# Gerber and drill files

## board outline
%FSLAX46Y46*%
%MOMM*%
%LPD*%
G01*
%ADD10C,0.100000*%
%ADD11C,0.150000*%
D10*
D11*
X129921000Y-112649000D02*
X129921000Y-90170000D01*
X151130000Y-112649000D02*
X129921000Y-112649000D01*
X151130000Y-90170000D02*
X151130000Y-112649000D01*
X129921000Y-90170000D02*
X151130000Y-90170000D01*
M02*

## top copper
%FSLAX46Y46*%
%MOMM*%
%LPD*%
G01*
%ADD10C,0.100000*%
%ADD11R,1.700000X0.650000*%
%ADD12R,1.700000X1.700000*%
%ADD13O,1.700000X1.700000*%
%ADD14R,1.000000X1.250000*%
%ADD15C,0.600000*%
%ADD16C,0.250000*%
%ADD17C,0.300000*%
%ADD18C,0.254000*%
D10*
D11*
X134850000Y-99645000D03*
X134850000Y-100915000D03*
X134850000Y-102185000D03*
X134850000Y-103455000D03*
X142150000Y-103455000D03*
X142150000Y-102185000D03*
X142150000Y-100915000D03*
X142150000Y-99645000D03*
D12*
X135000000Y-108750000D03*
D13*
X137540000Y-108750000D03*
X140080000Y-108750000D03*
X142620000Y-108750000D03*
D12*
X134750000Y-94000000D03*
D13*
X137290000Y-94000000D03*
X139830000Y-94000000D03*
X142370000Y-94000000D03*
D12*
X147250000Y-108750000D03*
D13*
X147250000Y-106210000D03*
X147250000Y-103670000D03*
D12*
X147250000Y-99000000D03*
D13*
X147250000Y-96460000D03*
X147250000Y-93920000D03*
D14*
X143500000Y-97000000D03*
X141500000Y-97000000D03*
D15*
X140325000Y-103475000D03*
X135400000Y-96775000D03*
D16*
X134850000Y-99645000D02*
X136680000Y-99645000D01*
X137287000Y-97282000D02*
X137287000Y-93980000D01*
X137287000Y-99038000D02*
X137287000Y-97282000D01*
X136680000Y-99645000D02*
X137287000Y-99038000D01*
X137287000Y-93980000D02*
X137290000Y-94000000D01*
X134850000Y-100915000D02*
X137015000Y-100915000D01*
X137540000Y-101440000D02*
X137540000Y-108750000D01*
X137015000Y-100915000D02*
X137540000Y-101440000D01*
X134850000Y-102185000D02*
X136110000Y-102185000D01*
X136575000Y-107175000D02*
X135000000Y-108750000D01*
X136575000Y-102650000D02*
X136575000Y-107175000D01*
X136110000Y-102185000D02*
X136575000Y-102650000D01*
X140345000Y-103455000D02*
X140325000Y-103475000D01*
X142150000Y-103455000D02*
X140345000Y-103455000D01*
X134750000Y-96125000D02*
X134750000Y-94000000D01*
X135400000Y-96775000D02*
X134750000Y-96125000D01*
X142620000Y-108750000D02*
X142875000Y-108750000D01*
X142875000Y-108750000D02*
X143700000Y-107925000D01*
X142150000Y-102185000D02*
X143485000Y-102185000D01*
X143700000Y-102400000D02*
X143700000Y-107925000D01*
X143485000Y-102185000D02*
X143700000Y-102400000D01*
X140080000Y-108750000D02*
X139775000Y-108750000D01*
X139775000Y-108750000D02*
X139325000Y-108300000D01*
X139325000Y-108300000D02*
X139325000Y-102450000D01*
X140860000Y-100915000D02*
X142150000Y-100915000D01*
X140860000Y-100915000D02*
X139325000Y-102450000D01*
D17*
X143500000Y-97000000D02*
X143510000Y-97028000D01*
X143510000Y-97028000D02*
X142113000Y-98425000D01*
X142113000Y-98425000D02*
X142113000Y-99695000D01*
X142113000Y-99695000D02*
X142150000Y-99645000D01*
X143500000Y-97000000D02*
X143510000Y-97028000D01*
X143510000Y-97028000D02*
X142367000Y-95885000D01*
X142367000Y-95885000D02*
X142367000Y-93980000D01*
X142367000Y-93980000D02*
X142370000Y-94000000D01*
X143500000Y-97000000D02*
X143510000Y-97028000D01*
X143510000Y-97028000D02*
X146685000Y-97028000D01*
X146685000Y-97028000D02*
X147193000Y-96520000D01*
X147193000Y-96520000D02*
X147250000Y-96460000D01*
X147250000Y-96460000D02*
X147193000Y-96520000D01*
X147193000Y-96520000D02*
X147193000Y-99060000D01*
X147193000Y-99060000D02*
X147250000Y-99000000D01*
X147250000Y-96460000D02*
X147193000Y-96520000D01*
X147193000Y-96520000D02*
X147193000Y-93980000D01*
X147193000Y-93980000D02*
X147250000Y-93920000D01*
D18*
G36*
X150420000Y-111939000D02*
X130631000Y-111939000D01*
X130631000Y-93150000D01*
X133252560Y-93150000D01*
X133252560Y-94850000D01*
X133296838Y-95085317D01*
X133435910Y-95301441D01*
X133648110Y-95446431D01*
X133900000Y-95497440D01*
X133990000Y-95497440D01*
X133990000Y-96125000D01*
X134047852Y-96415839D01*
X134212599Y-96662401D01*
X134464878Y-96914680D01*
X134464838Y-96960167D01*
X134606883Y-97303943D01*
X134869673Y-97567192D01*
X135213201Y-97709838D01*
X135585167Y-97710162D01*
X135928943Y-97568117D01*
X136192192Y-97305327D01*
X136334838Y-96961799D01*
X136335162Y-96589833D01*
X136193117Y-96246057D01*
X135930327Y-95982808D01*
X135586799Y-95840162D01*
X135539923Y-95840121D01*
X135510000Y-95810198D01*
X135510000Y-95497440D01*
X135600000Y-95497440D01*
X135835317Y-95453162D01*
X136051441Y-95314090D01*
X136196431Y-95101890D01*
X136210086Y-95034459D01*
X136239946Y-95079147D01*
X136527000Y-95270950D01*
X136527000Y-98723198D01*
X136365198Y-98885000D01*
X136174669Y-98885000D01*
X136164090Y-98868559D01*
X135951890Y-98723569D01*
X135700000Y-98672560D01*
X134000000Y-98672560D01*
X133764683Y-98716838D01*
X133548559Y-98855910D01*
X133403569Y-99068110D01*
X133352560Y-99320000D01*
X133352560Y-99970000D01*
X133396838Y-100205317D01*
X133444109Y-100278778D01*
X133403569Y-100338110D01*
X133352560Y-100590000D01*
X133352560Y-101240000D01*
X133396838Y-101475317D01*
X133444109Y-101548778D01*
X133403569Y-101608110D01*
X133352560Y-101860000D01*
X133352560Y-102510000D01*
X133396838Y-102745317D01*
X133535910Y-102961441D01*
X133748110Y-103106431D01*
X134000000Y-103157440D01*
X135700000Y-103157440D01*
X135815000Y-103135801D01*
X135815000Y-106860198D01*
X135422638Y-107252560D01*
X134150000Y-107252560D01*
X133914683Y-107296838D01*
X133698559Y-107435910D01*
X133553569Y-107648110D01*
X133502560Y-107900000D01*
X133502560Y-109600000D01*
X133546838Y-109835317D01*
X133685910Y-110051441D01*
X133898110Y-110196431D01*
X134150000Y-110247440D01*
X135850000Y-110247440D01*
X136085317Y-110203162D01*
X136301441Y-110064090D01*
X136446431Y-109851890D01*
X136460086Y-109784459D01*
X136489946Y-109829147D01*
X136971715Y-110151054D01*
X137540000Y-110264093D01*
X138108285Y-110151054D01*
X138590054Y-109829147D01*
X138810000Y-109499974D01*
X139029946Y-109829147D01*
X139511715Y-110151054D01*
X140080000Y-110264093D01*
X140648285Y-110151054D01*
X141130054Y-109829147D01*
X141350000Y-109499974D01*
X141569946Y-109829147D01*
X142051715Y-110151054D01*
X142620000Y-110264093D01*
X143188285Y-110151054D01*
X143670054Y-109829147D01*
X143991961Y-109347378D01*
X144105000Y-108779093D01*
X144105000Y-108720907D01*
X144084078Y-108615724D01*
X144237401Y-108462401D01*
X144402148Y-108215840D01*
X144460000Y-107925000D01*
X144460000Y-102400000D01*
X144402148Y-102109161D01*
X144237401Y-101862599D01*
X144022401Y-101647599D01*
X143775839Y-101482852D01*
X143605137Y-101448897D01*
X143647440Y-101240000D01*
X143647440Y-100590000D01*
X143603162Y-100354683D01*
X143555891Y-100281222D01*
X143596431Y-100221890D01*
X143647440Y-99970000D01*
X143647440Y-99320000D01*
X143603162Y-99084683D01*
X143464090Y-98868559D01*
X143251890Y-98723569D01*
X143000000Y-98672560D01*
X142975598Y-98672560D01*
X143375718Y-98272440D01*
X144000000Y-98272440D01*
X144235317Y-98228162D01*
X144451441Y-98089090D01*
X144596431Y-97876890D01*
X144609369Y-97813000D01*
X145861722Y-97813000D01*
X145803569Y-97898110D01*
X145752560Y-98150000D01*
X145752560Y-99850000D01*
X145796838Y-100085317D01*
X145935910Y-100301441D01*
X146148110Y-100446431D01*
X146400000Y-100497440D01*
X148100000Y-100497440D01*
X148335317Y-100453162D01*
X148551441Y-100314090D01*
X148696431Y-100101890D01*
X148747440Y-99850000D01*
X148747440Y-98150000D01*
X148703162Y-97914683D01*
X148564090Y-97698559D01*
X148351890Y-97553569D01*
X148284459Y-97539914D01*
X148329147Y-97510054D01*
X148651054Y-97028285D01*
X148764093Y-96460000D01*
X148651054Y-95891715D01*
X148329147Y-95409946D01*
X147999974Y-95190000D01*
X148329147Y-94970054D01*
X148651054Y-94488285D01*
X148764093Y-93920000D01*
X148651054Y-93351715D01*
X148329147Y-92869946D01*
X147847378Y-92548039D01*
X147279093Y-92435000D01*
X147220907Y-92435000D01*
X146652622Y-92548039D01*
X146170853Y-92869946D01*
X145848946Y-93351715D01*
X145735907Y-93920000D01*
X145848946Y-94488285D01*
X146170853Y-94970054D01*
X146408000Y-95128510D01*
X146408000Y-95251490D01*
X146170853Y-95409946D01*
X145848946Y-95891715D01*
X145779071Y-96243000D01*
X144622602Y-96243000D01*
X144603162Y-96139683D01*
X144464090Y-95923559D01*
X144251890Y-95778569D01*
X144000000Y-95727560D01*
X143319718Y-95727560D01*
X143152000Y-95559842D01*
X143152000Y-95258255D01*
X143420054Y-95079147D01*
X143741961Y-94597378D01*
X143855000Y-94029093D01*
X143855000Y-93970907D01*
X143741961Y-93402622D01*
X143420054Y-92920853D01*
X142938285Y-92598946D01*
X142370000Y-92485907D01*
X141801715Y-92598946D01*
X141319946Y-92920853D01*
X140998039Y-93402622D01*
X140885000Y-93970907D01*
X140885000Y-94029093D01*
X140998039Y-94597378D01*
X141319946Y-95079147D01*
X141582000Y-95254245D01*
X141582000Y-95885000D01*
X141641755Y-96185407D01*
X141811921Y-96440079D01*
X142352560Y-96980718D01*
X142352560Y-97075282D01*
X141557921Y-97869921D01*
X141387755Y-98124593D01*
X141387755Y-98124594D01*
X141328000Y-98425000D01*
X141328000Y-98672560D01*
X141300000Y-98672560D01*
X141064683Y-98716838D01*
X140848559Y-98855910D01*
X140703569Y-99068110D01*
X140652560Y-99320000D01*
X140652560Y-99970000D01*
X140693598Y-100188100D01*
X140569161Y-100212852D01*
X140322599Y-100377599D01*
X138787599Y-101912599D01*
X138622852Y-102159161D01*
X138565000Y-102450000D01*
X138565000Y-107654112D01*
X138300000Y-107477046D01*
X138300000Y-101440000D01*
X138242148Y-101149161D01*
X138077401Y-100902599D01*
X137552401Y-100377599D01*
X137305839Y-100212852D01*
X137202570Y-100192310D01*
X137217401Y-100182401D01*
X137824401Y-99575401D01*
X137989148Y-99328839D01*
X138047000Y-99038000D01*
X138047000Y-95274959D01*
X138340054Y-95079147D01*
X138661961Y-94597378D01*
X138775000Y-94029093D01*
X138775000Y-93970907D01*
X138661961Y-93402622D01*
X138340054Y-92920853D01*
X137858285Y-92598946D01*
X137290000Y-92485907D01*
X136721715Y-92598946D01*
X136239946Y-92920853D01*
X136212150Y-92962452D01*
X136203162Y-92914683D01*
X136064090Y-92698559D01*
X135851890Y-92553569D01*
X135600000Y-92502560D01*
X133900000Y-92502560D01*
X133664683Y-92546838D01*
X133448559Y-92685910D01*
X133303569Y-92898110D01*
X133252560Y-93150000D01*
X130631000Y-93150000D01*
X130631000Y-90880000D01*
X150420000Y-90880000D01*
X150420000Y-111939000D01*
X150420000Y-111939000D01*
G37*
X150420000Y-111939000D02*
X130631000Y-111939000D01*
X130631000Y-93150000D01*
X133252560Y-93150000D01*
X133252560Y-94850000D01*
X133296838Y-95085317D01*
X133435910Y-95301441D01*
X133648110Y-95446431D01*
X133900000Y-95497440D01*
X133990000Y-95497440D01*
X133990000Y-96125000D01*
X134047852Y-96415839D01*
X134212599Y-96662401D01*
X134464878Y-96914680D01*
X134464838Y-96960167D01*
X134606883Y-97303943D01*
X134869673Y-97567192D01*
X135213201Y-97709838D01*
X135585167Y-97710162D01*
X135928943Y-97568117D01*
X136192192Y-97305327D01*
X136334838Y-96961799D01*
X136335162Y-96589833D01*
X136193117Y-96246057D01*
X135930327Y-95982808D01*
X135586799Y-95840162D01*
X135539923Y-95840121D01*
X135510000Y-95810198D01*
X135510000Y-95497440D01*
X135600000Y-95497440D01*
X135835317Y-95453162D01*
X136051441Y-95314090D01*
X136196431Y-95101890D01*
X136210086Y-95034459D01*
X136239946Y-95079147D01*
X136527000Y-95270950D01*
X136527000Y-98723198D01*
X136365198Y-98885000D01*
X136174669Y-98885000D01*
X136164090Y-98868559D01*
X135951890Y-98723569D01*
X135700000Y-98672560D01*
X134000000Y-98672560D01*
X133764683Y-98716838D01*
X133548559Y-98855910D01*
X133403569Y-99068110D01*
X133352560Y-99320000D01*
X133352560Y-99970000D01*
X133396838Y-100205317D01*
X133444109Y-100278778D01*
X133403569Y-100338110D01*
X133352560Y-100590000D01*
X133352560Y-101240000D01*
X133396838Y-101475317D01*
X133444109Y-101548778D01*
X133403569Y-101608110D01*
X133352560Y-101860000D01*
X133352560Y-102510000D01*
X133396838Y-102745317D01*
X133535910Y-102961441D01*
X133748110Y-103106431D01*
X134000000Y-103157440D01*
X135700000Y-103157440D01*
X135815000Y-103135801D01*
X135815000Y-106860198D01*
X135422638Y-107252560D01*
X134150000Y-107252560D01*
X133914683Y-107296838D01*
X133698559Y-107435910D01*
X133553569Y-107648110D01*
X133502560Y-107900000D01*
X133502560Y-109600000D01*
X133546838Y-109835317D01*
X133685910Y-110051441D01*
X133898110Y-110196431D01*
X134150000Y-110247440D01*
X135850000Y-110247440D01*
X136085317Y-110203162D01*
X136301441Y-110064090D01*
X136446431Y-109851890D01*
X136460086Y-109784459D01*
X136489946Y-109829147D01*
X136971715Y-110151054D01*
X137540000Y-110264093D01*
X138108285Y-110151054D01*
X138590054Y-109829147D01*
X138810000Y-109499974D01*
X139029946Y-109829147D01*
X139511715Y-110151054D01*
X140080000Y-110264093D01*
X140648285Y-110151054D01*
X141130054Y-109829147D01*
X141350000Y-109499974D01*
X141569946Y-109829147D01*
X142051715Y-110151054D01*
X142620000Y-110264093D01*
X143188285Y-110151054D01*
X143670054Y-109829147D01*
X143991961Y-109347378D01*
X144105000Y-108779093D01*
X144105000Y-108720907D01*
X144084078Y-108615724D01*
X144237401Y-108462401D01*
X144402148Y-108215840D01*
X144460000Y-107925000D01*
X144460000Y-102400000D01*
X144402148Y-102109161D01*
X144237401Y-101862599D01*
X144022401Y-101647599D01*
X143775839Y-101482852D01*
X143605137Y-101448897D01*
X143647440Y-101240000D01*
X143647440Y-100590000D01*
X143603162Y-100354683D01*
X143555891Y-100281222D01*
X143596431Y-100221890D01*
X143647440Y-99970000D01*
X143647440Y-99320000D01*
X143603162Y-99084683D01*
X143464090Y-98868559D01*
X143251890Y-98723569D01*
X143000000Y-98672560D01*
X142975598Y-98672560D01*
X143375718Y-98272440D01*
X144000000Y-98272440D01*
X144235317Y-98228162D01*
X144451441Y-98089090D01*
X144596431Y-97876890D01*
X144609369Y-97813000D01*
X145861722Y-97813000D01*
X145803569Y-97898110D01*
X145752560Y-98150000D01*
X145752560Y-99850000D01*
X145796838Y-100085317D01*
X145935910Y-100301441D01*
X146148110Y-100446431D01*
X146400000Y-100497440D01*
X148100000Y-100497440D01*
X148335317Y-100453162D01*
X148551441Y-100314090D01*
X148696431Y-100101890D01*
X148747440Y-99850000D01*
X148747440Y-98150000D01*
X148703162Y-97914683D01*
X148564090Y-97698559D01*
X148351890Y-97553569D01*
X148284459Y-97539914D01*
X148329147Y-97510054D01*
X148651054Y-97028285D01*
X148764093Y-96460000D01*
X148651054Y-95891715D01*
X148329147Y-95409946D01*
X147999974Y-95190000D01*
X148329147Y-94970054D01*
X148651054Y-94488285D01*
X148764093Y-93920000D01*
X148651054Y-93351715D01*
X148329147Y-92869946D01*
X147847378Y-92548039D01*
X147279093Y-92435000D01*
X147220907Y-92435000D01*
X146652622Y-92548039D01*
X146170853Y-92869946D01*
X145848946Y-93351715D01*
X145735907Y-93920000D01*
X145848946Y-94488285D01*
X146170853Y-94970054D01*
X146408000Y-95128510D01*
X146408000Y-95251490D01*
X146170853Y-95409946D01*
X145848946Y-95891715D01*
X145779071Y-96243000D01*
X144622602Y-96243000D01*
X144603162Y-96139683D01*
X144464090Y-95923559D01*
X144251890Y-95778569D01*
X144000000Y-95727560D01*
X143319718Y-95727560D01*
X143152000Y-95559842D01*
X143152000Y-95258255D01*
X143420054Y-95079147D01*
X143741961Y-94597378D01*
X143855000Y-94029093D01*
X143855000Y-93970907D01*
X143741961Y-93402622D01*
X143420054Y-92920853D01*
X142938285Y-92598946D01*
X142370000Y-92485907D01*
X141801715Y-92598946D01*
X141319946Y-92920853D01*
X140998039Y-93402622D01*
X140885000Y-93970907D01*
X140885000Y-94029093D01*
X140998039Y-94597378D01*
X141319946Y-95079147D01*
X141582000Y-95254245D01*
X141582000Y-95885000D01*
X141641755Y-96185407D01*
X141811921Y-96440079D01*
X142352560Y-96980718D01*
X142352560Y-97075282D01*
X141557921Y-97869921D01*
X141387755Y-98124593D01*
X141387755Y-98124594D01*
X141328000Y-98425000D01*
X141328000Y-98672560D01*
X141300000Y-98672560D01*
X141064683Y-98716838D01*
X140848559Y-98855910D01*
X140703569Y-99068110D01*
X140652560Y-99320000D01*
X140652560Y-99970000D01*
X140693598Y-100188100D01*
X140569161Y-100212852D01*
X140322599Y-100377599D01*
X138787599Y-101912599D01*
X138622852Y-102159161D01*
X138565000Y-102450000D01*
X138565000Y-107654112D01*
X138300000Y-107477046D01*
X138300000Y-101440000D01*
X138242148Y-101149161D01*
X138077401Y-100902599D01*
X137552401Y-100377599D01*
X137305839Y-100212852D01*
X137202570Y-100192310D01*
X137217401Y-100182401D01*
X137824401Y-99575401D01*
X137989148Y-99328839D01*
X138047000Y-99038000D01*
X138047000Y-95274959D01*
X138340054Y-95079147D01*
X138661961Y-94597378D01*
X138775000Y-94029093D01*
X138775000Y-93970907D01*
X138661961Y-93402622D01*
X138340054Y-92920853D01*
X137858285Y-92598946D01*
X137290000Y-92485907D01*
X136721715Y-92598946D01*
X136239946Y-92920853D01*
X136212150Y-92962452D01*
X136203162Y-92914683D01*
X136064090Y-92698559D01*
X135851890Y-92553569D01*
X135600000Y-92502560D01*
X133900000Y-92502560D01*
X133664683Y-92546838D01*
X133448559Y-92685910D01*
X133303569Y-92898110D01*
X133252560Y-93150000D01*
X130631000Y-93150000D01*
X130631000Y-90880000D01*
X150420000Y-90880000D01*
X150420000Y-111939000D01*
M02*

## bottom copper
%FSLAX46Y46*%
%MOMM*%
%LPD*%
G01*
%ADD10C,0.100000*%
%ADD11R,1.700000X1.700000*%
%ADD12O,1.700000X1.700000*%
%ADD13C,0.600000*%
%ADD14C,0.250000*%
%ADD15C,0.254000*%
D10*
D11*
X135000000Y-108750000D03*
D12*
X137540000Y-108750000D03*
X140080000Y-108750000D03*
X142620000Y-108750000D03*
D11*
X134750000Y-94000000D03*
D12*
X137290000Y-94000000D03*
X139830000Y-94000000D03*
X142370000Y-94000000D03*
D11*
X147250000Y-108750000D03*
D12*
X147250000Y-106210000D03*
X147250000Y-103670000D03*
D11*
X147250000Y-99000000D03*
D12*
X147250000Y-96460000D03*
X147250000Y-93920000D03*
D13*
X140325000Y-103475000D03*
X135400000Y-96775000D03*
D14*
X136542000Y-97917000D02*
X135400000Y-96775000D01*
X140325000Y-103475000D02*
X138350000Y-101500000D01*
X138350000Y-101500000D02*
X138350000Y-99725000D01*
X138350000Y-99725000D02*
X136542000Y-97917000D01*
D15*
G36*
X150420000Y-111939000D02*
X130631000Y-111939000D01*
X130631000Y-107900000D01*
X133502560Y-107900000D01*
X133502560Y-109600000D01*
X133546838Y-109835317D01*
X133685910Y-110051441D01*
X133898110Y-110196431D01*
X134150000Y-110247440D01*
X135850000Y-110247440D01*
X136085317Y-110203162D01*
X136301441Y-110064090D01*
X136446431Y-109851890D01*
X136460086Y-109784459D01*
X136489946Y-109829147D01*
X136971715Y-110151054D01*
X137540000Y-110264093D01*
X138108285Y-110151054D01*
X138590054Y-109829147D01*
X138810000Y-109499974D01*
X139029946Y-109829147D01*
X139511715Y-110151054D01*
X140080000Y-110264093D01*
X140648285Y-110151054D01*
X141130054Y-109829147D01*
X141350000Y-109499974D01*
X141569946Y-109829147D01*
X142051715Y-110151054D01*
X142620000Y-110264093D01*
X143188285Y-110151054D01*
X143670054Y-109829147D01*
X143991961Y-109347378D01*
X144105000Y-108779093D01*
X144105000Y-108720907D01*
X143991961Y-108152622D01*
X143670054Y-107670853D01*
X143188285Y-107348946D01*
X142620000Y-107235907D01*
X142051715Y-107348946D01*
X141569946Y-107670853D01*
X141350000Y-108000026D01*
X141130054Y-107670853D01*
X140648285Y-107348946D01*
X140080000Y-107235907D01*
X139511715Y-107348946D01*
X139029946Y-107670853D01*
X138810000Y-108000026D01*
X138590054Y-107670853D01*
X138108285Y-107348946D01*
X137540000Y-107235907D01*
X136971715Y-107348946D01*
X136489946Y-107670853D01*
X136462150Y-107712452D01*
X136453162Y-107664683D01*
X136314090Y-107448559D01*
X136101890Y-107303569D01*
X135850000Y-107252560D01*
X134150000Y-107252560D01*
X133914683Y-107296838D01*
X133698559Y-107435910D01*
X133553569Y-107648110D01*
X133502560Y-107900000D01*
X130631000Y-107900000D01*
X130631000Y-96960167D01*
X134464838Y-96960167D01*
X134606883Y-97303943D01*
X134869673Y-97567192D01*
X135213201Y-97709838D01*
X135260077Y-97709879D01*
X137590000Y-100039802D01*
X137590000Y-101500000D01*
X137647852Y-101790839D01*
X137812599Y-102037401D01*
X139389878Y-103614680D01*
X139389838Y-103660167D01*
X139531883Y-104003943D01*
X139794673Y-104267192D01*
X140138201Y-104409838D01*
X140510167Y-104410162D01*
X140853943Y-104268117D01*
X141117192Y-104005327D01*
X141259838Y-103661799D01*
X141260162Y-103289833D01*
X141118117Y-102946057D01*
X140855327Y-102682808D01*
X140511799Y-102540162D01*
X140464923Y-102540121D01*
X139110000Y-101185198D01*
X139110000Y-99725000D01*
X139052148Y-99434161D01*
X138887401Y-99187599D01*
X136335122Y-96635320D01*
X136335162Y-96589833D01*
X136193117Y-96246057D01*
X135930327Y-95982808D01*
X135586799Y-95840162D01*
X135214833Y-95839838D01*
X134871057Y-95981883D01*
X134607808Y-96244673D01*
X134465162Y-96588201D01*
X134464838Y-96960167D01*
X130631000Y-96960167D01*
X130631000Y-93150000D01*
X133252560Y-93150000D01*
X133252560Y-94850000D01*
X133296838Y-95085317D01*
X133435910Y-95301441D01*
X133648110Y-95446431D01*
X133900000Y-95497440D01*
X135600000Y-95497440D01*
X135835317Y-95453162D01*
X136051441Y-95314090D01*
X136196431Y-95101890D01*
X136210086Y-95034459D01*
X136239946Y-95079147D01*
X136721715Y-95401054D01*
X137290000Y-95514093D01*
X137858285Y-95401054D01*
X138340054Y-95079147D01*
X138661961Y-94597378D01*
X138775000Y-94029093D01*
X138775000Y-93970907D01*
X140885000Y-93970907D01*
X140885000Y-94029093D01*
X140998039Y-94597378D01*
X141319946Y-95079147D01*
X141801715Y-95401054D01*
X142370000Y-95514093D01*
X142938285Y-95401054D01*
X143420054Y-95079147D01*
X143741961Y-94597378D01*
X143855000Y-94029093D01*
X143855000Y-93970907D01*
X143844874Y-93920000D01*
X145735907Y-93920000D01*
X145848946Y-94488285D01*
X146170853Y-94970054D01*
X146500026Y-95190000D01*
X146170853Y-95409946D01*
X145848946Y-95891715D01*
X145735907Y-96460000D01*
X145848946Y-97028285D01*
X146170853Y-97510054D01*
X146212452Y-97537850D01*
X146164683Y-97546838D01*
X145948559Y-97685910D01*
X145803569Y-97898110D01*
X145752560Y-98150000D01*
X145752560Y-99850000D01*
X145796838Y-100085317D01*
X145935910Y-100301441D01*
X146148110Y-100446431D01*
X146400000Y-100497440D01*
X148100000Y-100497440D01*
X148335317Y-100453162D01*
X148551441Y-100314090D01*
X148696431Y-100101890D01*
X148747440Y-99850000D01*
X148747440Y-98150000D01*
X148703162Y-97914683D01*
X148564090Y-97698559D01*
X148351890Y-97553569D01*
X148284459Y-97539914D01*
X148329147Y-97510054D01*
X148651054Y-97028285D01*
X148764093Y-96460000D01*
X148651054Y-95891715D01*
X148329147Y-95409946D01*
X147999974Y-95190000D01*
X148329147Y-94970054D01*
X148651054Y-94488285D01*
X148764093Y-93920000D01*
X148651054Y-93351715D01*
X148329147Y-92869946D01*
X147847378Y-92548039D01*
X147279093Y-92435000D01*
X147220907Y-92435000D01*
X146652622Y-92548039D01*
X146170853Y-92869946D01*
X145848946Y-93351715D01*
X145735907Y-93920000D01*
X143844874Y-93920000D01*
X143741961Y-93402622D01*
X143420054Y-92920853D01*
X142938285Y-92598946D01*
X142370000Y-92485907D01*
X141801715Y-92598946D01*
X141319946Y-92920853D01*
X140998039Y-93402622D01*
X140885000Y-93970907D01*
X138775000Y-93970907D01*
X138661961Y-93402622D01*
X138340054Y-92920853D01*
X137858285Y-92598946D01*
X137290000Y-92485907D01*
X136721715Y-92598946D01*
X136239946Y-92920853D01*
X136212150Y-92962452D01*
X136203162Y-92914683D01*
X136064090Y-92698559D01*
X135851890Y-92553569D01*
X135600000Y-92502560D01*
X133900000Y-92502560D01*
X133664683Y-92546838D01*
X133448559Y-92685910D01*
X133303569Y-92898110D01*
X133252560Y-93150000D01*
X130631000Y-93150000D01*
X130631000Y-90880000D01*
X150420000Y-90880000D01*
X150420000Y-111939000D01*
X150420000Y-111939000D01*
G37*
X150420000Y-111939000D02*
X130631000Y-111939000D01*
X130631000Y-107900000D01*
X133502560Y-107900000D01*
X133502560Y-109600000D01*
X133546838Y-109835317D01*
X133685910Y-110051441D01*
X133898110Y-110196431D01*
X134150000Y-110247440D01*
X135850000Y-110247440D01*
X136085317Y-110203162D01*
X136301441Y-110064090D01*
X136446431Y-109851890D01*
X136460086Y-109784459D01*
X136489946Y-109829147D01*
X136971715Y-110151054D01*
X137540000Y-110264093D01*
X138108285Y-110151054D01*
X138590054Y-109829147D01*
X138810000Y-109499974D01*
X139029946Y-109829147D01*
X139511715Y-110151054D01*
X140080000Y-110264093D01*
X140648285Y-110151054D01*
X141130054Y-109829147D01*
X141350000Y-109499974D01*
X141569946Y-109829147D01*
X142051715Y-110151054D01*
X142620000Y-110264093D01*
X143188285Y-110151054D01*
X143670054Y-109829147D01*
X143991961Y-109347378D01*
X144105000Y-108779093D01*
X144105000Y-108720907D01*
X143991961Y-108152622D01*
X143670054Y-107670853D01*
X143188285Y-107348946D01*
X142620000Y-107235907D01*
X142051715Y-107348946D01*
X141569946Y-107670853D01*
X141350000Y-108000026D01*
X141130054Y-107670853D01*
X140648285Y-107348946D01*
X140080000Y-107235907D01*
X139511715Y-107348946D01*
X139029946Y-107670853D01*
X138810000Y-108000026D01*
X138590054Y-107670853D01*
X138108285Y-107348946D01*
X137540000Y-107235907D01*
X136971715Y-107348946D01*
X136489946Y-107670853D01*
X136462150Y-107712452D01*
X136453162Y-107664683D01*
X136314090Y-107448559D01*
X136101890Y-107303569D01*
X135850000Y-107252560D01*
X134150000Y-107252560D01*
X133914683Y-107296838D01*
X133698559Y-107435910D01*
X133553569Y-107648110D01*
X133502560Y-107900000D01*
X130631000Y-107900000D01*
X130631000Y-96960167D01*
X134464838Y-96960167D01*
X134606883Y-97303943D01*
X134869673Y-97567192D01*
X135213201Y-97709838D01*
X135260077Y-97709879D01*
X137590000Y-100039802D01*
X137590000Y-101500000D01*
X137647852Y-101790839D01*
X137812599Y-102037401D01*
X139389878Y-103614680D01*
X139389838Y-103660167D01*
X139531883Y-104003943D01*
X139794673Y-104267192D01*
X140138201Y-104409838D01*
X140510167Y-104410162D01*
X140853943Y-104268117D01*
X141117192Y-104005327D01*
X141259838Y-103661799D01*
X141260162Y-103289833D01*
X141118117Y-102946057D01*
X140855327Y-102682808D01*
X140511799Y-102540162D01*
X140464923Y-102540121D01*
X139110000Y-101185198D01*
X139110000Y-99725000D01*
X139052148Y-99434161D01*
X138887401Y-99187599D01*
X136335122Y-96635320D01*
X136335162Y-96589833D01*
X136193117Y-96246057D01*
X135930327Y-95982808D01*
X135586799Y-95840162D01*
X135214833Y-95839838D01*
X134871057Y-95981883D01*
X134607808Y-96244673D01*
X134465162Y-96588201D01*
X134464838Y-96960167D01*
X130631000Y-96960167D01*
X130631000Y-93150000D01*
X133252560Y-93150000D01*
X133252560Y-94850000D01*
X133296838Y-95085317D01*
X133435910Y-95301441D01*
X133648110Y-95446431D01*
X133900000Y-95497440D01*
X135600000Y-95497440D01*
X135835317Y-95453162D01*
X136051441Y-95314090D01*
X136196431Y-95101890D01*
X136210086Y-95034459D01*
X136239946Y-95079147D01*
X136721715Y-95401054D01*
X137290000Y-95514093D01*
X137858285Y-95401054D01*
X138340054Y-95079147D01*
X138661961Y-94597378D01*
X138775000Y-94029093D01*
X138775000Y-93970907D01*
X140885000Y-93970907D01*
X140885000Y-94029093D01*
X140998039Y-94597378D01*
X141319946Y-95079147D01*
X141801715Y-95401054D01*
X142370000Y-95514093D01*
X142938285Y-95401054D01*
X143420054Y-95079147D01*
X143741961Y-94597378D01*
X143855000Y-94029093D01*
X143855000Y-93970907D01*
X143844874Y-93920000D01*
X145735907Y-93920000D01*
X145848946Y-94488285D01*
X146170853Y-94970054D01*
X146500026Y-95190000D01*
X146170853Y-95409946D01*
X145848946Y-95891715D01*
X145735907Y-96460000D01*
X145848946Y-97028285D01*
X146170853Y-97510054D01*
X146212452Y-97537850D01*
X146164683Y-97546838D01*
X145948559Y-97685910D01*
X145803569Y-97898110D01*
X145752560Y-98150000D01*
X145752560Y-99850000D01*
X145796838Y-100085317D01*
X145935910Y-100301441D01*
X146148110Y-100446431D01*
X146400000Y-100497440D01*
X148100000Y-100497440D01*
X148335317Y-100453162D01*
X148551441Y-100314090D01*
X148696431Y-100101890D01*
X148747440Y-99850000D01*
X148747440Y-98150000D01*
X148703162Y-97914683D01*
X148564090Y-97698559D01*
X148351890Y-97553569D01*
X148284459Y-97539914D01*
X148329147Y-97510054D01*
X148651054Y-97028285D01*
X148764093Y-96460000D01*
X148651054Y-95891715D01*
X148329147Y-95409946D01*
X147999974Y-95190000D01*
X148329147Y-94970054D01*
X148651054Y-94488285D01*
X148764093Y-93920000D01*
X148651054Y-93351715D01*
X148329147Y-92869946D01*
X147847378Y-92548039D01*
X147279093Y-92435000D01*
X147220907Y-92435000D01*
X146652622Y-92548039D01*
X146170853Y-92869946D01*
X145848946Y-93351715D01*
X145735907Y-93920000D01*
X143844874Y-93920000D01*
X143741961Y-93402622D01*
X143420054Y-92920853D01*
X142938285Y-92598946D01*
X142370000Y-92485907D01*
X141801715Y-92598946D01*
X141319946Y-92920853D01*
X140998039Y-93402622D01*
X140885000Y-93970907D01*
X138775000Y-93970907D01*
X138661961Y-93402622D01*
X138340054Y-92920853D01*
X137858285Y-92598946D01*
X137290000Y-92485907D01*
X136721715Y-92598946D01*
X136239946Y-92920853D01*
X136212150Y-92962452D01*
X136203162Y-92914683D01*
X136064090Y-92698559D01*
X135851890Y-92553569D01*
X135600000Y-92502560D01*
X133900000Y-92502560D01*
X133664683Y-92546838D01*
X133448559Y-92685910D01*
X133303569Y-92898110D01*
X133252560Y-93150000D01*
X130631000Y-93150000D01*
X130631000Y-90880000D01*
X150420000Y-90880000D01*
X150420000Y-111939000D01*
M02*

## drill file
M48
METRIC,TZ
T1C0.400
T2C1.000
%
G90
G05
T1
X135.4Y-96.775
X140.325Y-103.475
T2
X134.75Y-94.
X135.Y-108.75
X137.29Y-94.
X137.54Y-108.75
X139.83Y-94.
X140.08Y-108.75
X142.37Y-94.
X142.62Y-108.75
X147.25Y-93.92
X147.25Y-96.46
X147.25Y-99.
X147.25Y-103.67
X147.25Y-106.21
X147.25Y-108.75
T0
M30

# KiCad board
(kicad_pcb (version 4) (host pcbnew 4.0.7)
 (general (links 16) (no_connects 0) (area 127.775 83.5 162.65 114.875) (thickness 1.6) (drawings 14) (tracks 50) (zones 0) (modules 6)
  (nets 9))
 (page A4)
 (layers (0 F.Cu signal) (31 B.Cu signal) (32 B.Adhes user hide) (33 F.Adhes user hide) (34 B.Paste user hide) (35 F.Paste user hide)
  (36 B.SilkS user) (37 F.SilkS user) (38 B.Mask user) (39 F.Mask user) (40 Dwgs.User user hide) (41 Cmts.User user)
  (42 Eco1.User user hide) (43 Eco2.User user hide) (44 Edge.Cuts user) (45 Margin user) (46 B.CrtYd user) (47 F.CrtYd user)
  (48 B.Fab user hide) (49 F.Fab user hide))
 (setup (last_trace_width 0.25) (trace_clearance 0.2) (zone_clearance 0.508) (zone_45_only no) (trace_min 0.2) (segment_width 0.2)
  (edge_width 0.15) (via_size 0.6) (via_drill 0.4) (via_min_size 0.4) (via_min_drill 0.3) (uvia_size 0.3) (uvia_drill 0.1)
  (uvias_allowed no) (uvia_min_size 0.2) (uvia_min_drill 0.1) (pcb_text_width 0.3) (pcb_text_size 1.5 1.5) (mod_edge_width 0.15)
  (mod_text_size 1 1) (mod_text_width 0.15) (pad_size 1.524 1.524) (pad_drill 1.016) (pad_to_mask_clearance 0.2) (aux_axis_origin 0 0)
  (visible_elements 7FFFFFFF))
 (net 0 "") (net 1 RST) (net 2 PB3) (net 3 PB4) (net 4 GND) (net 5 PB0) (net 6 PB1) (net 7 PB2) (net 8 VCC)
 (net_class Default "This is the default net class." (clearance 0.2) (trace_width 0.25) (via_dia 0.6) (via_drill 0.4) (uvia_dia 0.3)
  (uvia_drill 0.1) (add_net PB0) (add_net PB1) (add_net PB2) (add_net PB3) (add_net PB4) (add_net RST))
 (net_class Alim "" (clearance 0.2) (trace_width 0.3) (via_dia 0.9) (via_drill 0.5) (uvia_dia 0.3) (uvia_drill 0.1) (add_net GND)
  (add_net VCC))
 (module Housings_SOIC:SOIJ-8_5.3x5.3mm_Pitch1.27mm (layer F.Cu) (at 138.5 101.55)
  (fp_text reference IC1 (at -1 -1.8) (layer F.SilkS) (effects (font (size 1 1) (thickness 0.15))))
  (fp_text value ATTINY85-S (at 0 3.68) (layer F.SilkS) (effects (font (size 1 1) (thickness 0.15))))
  (pad 1 smd rect (at -3.65 -1.905) (size 1.7 0.65) (layers F.Cu F.Paste F.Mask) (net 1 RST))
  (pad 2 smd rect (at -3.65 -0.635) (size 1.7 0.65) (layers F.Cu F.Paste F.Mask) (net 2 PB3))
  (pad 3 smd rect (at -3.65 0.635) (size 1.7 0.65) (layers F.Cu F.Paste F.Mask) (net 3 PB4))
  (pad 4 smd rect (at -3.65 1.905) (size 1.7 0.65) (layers F.Cu F.Paste F.Mask) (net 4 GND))
  (pad 5 smd rect (at 3.65 1.905) (size 1.7 0.65) (layers F.Cu F.Paste F.Mask) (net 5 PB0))
  (pad 6 smd rect (at 3.65 0.635) (size 1.7 0.65) (layers F.Cu F.Paste F.Mask) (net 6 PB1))
  (pad 7 smd rect (at 3.65 -0.635) (size 1.7 0.65) (layers F.Cu F.Paste F.Mask) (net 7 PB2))
  (pad 8 smd rect (at 3.65 -1.905) (size 1.7 0.65) (layers F.Cu F.Paste F.Mask) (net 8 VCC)))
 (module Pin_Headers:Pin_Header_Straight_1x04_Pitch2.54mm (layer F.Cu) (at 135 108.75 90)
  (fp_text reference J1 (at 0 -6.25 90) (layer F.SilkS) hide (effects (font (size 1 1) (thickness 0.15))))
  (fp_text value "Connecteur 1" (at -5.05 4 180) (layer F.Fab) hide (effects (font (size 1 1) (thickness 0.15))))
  (pad 1 thru_hole rect (at 0 0 90) (size 1.7 1.7) (drill 1) (layers *.Cu *.Mask) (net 3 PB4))
  (pad 2 thru_hole oval (at 0 2.54 90) (size 1.7 1.7) (drill 1) (layers *.Cu *.Mask) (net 2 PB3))
  (pad 3 thru_hole oval (at 0 5.08 90) (size 1.7 1.7) (drill 1) (layers *.Cu *.Mask) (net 7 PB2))
  (pad 4 thru_hole oval (at 0 7.62 90) (size 1.7 1.7) (drill 1) (layers *.Cu *.Mask) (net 6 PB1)))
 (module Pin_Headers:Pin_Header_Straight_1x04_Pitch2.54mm (layer F.Cu) (at 134.75 94 90)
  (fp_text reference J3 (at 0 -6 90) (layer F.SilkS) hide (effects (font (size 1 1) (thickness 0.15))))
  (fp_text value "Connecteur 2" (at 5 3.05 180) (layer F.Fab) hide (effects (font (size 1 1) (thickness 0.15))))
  (pad 1 thru_hole rect (at 0 0 90) (size 1.7 1.7) (drill 1) (layers *.Cu *.Mask) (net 5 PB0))
  (pad 2 thru_hole oval (at 0 2.54 90) (size 1.7 1.7) (drill 1) (layers *.Cu *.Mask) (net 1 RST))
  (pad 3 thru_hole oval (at 0 5.08 90) (size 1.7 1.7) (drill 1) (layers *.Cu *.Mask) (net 4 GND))
  (pad 4 thru_hole oval (at 0 7.62 90) (size 1.7 1.7) (drill 1) (layers *.Cu *.Mask) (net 8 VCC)))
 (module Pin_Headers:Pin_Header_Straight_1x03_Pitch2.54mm (layer F.Cu) (at 147.25 108.75 180)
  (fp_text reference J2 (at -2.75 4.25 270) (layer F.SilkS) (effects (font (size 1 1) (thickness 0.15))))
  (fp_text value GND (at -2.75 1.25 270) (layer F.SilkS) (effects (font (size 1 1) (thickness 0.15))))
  (pad 1 thru_hole rect (at 0 0 180) (size 1.7 1.7) (drill 1) (layers *.Cu *.Mask) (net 4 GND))
  (pad 2 thru_hole oval (at 0 2.54 180) (size 1.7 1.7) (drill 1) (layers *.Cu *.Mask) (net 4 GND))
  (pad 3 thru_hole oval (at 0 5.08 180) (size 1.7 1.7) (drill 1) (layers *.Cu *.Mask) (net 4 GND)))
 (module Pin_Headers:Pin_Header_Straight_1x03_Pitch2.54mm (layer F.Cu) (at 147.25 99 180)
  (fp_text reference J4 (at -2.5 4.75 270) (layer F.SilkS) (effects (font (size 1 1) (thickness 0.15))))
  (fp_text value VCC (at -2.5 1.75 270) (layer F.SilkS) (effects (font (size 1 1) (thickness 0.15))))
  (pad 1 thru_hole rect (at 0 0 180) (size 1.7 1.7) (drill 1) (layers *.Cu *.Mask) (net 8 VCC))
  (pad 2 thru_hole oval (at 0 2.54 180) (size 1.7 1.7) (drill 1) (layers *.Cu *.Mask) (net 8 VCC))
  (pad 3 thru_hole oval (at 0 5.08 180) (size 1.7 1.7) (drill 1) (layers *.Cu *.Mask) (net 8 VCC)))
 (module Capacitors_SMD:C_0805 (layer F.Cu) (at 142.5 97 180)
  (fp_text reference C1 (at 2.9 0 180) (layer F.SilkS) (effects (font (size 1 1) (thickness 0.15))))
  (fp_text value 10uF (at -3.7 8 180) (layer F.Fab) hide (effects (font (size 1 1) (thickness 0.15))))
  (pad 1 smd rect (at -1 0 180) (size 1 1.25) (layers F.Cu F.Paste F.Mask) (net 8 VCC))
  (pad 2 smd rect (at 1 0 180) (size 1 1.25) (layers F.Cu F.Paste F.Mask) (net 4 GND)))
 (gr_line (start 129.921 112.649) (end 129.921 90.17) (angle 90) (layer Edge.Cuts) (width 0.15))
 (gr_line (start 151.13 112.649) (end 129.921 112.649) (angle 90) (layer Edge.Cuts) (width 0.15))
 (gr_line (start 151.13 90.17) (end 151.13 112.649) (angle 90) (layer Edge.Cuts) (width 0.15))
 (gr_line (start 129.921 90.17) (end 151.13 90.17) (angle 90) (layer Edge.Cuts) (width 0.15))
 (segment (start 134.85 99.645) (end 136.68 99.645) (width 0.25) (layer F.Cu) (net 1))
 (segment (start 137.287 97.282) (end 137.287 93.98) (width 0.25) (layer F.Cu) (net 1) (status 80000))
 (segment (start 137.287 99.038) (end 137.287 97.282) (width 0.25) (layer F.Cu) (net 1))
 (segment (start 136.68 99.645) (end 137.287 99.038) (width 0.25) (layer F.Cu) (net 1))
 (segment (start 137.287 93.98) (end 137.29 94) (width 0.25) (layer F.Cu) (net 1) (status 80000))
 (segment (start 134.85 100.915) (end 137.015 100.915) (width 0.25) (layer F.Cu) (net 2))
 (segment (start 137.54 101.44) (end 137.54 108.75) (width 0.25) (layer F.Cu) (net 2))
 (segment (start 137.015 100.915) (end 137.54 101.44) (width 0.25) (layer F.Cu) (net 2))
 (segment (start 134.85 102.185) (end 136.11 102.185) (width 0.25) (layer F.Cu) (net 3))
 (segment (start 136.575 107.175) (end 135 108.75) (width 0.25) (layer F.Cu) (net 3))
 (segment (start 136.575 102.65) (end 136.575 107.175) (width 0.25) (layer F.Cu) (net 3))
 (segment (start 136.11 102.185) (end 136.575 102.65) (width 0.25) (layer F.Cu) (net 3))
 (segment (start 136.542 97.917) (end 135.4 96.775) (width 0.25) (layer B.Cu) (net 5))
 (segment (start 140.345 103.455) (end 140.325 103.475) (width 0.25) (layer F.Cu) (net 5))
 (via (at 140.325 103.475) (size 0.6) (drill 0.4) (layers F.Cu B.Cu) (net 5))
 (segment (start 140.325 103.475) (end 138.35 101.5) (width 0.25) (layer B.Cu) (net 5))
 (segment (start 138.35 101.5) (end 138.35 99.725) (width 0.25) (layer B.Cu) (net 5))
 (segment (start 138.35 99.725) (end 136.542 97.917) (width 0.25) (layer B.Cu) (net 5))
 (segment (start 142.15 103.455) (end 140.345 103.455) (width 0.25) (layer F.Cu) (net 5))
 (segment (start 134.75 96.125) (end 134.75 94) (width 0.25) (layer F.Cu) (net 5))
 (segment (start 135.4 96.775) (end 134.75 96.125) (width 0.25) (layer F.Cu) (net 5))
 (via (at 135.4 96.775) (size 0.6) (drill 0.4) (layers F.Cu B.Cu) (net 5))
 (segment (start 142.62 108.75) (end 142.875 108.75) (width 0.25) (layer F.Cu) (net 6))
 (segment (start 142.875 108.75) (end 143.7 107.925) (width 0.25) (layer F.Cu) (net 6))
 (segment (start 142.15 102.185) (end 143.485 102.185) (width 0.25) (layer F.Cu) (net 6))
 (segment (start 143.7 102.4) (end 143.7 107.925) (width 0.25) (layer F.Cu) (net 6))
 (segment (start 143.485 102.185) (end 143.7 102.4) (width 0.25) (layer F.Cu) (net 6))
 (segment (start 140.08 108.75) (end 139.775 108.75) (width 0.25) (layer F.Cu) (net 7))
 (segment (start 139.775 108.75) (end 139.325 108.3) (width 0.25) (layer F.Cu) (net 7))
 (segment (start 139.325 108.3) (end 139.325 102.45) (width 0.25) (layer F.Cu) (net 7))
 (segment (start 140.86 100.915) (end 142.15 100.915) (width 0.25) (layer F.Cu) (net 7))
 (segment (start 140.86 100.915) (end 139.325 102.45) (width 0.25) (layer F.Cu) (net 7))
 (segment (start 143.5 97) (end 143.51 97.028) (width 0.3) (layer F.Cu) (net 8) (status 80000))
 (segment (start 143.51 97.028) (end 142.113 98.425) (width 0.3) (layer F.Cu) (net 8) (status 80000))
 (segment (start 142.113 98.425) (end 142.113 99.695) (width 0.3) (layer F.Cu) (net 8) (status 80000))
 (segment (start 142.113 99.695) (end 142.15 99.645) (width 0.3) (layer F.Cu) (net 8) (status 80000))
 (segment (start 143.5 97) (end 143.51 97.028) (width 0.3) (layer F.Cu) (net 8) (status 80000))
 (segment (start 143.51 97.028) (end 142.367 95.885) (width 0.3) (layer F.Cu) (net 8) (status 80000))
 (segment (start 142.367 95.885) (end 142.367 93.98) (width 0.3) (layer F.Cu) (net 8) (status 80000))
 (segment (start 142.367 93.98) (end 142.37 94) (width 0.3) (layer F.Cu) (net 8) (status 80000))
 (segment (start 143.5 97) (end 143.51 97.028) (width 0.3) (layer F.Cu) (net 8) (status 80000))
 (segment (start 143.51 97.028) (end 146.685 97.028) (width 0.3) (layer F.Cu) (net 8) (status 80000))
 (segment (start 146.685 97.028) (end 147.193 96.52) (width 0.3) (layer F.Cu) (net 8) (status 80000))
 (segment (start 147.193 96.52) (end 147.25 96.46) (width 0.3) (layer F.Cu) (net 8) (status 80000))
 (segment (start 147.25 96.46) (end 147.193 96.52) (width 0.3) (layer F.Cu) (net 8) (status 80000))
 (segment (start 147.193 96.52) (end 147.193 99.06) (width 0.3) (layer F.Cu) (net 8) (status 80000))
 (segment (start 147.193 99.06) (end 147.25 99) (width 0.3) (layer F.Cu) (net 8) (status 80000))
 (segment (start 147.25 96.46) (end 147.193 96.52) (width 0.3) (layer F.Cu) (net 8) (status 80000))
 (segment (start 147.193 96.52) (end 147.193 93.98) (width 0.3) (layer F.Cu) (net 8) (status 80000))
 (segment (start 147.193 93.98) (end 147.25 93.92) (width 0.3) (layer F.Cu) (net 8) (status 80000))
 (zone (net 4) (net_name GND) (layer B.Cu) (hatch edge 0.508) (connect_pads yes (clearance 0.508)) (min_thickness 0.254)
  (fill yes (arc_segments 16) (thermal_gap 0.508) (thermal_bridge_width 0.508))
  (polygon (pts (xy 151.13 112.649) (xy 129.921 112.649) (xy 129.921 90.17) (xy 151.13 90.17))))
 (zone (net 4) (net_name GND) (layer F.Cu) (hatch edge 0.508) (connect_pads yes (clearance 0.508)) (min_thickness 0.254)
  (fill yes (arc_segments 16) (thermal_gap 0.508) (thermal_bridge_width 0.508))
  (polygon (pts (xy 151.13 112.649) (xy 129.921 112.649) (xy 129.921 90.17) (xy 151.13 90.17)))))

